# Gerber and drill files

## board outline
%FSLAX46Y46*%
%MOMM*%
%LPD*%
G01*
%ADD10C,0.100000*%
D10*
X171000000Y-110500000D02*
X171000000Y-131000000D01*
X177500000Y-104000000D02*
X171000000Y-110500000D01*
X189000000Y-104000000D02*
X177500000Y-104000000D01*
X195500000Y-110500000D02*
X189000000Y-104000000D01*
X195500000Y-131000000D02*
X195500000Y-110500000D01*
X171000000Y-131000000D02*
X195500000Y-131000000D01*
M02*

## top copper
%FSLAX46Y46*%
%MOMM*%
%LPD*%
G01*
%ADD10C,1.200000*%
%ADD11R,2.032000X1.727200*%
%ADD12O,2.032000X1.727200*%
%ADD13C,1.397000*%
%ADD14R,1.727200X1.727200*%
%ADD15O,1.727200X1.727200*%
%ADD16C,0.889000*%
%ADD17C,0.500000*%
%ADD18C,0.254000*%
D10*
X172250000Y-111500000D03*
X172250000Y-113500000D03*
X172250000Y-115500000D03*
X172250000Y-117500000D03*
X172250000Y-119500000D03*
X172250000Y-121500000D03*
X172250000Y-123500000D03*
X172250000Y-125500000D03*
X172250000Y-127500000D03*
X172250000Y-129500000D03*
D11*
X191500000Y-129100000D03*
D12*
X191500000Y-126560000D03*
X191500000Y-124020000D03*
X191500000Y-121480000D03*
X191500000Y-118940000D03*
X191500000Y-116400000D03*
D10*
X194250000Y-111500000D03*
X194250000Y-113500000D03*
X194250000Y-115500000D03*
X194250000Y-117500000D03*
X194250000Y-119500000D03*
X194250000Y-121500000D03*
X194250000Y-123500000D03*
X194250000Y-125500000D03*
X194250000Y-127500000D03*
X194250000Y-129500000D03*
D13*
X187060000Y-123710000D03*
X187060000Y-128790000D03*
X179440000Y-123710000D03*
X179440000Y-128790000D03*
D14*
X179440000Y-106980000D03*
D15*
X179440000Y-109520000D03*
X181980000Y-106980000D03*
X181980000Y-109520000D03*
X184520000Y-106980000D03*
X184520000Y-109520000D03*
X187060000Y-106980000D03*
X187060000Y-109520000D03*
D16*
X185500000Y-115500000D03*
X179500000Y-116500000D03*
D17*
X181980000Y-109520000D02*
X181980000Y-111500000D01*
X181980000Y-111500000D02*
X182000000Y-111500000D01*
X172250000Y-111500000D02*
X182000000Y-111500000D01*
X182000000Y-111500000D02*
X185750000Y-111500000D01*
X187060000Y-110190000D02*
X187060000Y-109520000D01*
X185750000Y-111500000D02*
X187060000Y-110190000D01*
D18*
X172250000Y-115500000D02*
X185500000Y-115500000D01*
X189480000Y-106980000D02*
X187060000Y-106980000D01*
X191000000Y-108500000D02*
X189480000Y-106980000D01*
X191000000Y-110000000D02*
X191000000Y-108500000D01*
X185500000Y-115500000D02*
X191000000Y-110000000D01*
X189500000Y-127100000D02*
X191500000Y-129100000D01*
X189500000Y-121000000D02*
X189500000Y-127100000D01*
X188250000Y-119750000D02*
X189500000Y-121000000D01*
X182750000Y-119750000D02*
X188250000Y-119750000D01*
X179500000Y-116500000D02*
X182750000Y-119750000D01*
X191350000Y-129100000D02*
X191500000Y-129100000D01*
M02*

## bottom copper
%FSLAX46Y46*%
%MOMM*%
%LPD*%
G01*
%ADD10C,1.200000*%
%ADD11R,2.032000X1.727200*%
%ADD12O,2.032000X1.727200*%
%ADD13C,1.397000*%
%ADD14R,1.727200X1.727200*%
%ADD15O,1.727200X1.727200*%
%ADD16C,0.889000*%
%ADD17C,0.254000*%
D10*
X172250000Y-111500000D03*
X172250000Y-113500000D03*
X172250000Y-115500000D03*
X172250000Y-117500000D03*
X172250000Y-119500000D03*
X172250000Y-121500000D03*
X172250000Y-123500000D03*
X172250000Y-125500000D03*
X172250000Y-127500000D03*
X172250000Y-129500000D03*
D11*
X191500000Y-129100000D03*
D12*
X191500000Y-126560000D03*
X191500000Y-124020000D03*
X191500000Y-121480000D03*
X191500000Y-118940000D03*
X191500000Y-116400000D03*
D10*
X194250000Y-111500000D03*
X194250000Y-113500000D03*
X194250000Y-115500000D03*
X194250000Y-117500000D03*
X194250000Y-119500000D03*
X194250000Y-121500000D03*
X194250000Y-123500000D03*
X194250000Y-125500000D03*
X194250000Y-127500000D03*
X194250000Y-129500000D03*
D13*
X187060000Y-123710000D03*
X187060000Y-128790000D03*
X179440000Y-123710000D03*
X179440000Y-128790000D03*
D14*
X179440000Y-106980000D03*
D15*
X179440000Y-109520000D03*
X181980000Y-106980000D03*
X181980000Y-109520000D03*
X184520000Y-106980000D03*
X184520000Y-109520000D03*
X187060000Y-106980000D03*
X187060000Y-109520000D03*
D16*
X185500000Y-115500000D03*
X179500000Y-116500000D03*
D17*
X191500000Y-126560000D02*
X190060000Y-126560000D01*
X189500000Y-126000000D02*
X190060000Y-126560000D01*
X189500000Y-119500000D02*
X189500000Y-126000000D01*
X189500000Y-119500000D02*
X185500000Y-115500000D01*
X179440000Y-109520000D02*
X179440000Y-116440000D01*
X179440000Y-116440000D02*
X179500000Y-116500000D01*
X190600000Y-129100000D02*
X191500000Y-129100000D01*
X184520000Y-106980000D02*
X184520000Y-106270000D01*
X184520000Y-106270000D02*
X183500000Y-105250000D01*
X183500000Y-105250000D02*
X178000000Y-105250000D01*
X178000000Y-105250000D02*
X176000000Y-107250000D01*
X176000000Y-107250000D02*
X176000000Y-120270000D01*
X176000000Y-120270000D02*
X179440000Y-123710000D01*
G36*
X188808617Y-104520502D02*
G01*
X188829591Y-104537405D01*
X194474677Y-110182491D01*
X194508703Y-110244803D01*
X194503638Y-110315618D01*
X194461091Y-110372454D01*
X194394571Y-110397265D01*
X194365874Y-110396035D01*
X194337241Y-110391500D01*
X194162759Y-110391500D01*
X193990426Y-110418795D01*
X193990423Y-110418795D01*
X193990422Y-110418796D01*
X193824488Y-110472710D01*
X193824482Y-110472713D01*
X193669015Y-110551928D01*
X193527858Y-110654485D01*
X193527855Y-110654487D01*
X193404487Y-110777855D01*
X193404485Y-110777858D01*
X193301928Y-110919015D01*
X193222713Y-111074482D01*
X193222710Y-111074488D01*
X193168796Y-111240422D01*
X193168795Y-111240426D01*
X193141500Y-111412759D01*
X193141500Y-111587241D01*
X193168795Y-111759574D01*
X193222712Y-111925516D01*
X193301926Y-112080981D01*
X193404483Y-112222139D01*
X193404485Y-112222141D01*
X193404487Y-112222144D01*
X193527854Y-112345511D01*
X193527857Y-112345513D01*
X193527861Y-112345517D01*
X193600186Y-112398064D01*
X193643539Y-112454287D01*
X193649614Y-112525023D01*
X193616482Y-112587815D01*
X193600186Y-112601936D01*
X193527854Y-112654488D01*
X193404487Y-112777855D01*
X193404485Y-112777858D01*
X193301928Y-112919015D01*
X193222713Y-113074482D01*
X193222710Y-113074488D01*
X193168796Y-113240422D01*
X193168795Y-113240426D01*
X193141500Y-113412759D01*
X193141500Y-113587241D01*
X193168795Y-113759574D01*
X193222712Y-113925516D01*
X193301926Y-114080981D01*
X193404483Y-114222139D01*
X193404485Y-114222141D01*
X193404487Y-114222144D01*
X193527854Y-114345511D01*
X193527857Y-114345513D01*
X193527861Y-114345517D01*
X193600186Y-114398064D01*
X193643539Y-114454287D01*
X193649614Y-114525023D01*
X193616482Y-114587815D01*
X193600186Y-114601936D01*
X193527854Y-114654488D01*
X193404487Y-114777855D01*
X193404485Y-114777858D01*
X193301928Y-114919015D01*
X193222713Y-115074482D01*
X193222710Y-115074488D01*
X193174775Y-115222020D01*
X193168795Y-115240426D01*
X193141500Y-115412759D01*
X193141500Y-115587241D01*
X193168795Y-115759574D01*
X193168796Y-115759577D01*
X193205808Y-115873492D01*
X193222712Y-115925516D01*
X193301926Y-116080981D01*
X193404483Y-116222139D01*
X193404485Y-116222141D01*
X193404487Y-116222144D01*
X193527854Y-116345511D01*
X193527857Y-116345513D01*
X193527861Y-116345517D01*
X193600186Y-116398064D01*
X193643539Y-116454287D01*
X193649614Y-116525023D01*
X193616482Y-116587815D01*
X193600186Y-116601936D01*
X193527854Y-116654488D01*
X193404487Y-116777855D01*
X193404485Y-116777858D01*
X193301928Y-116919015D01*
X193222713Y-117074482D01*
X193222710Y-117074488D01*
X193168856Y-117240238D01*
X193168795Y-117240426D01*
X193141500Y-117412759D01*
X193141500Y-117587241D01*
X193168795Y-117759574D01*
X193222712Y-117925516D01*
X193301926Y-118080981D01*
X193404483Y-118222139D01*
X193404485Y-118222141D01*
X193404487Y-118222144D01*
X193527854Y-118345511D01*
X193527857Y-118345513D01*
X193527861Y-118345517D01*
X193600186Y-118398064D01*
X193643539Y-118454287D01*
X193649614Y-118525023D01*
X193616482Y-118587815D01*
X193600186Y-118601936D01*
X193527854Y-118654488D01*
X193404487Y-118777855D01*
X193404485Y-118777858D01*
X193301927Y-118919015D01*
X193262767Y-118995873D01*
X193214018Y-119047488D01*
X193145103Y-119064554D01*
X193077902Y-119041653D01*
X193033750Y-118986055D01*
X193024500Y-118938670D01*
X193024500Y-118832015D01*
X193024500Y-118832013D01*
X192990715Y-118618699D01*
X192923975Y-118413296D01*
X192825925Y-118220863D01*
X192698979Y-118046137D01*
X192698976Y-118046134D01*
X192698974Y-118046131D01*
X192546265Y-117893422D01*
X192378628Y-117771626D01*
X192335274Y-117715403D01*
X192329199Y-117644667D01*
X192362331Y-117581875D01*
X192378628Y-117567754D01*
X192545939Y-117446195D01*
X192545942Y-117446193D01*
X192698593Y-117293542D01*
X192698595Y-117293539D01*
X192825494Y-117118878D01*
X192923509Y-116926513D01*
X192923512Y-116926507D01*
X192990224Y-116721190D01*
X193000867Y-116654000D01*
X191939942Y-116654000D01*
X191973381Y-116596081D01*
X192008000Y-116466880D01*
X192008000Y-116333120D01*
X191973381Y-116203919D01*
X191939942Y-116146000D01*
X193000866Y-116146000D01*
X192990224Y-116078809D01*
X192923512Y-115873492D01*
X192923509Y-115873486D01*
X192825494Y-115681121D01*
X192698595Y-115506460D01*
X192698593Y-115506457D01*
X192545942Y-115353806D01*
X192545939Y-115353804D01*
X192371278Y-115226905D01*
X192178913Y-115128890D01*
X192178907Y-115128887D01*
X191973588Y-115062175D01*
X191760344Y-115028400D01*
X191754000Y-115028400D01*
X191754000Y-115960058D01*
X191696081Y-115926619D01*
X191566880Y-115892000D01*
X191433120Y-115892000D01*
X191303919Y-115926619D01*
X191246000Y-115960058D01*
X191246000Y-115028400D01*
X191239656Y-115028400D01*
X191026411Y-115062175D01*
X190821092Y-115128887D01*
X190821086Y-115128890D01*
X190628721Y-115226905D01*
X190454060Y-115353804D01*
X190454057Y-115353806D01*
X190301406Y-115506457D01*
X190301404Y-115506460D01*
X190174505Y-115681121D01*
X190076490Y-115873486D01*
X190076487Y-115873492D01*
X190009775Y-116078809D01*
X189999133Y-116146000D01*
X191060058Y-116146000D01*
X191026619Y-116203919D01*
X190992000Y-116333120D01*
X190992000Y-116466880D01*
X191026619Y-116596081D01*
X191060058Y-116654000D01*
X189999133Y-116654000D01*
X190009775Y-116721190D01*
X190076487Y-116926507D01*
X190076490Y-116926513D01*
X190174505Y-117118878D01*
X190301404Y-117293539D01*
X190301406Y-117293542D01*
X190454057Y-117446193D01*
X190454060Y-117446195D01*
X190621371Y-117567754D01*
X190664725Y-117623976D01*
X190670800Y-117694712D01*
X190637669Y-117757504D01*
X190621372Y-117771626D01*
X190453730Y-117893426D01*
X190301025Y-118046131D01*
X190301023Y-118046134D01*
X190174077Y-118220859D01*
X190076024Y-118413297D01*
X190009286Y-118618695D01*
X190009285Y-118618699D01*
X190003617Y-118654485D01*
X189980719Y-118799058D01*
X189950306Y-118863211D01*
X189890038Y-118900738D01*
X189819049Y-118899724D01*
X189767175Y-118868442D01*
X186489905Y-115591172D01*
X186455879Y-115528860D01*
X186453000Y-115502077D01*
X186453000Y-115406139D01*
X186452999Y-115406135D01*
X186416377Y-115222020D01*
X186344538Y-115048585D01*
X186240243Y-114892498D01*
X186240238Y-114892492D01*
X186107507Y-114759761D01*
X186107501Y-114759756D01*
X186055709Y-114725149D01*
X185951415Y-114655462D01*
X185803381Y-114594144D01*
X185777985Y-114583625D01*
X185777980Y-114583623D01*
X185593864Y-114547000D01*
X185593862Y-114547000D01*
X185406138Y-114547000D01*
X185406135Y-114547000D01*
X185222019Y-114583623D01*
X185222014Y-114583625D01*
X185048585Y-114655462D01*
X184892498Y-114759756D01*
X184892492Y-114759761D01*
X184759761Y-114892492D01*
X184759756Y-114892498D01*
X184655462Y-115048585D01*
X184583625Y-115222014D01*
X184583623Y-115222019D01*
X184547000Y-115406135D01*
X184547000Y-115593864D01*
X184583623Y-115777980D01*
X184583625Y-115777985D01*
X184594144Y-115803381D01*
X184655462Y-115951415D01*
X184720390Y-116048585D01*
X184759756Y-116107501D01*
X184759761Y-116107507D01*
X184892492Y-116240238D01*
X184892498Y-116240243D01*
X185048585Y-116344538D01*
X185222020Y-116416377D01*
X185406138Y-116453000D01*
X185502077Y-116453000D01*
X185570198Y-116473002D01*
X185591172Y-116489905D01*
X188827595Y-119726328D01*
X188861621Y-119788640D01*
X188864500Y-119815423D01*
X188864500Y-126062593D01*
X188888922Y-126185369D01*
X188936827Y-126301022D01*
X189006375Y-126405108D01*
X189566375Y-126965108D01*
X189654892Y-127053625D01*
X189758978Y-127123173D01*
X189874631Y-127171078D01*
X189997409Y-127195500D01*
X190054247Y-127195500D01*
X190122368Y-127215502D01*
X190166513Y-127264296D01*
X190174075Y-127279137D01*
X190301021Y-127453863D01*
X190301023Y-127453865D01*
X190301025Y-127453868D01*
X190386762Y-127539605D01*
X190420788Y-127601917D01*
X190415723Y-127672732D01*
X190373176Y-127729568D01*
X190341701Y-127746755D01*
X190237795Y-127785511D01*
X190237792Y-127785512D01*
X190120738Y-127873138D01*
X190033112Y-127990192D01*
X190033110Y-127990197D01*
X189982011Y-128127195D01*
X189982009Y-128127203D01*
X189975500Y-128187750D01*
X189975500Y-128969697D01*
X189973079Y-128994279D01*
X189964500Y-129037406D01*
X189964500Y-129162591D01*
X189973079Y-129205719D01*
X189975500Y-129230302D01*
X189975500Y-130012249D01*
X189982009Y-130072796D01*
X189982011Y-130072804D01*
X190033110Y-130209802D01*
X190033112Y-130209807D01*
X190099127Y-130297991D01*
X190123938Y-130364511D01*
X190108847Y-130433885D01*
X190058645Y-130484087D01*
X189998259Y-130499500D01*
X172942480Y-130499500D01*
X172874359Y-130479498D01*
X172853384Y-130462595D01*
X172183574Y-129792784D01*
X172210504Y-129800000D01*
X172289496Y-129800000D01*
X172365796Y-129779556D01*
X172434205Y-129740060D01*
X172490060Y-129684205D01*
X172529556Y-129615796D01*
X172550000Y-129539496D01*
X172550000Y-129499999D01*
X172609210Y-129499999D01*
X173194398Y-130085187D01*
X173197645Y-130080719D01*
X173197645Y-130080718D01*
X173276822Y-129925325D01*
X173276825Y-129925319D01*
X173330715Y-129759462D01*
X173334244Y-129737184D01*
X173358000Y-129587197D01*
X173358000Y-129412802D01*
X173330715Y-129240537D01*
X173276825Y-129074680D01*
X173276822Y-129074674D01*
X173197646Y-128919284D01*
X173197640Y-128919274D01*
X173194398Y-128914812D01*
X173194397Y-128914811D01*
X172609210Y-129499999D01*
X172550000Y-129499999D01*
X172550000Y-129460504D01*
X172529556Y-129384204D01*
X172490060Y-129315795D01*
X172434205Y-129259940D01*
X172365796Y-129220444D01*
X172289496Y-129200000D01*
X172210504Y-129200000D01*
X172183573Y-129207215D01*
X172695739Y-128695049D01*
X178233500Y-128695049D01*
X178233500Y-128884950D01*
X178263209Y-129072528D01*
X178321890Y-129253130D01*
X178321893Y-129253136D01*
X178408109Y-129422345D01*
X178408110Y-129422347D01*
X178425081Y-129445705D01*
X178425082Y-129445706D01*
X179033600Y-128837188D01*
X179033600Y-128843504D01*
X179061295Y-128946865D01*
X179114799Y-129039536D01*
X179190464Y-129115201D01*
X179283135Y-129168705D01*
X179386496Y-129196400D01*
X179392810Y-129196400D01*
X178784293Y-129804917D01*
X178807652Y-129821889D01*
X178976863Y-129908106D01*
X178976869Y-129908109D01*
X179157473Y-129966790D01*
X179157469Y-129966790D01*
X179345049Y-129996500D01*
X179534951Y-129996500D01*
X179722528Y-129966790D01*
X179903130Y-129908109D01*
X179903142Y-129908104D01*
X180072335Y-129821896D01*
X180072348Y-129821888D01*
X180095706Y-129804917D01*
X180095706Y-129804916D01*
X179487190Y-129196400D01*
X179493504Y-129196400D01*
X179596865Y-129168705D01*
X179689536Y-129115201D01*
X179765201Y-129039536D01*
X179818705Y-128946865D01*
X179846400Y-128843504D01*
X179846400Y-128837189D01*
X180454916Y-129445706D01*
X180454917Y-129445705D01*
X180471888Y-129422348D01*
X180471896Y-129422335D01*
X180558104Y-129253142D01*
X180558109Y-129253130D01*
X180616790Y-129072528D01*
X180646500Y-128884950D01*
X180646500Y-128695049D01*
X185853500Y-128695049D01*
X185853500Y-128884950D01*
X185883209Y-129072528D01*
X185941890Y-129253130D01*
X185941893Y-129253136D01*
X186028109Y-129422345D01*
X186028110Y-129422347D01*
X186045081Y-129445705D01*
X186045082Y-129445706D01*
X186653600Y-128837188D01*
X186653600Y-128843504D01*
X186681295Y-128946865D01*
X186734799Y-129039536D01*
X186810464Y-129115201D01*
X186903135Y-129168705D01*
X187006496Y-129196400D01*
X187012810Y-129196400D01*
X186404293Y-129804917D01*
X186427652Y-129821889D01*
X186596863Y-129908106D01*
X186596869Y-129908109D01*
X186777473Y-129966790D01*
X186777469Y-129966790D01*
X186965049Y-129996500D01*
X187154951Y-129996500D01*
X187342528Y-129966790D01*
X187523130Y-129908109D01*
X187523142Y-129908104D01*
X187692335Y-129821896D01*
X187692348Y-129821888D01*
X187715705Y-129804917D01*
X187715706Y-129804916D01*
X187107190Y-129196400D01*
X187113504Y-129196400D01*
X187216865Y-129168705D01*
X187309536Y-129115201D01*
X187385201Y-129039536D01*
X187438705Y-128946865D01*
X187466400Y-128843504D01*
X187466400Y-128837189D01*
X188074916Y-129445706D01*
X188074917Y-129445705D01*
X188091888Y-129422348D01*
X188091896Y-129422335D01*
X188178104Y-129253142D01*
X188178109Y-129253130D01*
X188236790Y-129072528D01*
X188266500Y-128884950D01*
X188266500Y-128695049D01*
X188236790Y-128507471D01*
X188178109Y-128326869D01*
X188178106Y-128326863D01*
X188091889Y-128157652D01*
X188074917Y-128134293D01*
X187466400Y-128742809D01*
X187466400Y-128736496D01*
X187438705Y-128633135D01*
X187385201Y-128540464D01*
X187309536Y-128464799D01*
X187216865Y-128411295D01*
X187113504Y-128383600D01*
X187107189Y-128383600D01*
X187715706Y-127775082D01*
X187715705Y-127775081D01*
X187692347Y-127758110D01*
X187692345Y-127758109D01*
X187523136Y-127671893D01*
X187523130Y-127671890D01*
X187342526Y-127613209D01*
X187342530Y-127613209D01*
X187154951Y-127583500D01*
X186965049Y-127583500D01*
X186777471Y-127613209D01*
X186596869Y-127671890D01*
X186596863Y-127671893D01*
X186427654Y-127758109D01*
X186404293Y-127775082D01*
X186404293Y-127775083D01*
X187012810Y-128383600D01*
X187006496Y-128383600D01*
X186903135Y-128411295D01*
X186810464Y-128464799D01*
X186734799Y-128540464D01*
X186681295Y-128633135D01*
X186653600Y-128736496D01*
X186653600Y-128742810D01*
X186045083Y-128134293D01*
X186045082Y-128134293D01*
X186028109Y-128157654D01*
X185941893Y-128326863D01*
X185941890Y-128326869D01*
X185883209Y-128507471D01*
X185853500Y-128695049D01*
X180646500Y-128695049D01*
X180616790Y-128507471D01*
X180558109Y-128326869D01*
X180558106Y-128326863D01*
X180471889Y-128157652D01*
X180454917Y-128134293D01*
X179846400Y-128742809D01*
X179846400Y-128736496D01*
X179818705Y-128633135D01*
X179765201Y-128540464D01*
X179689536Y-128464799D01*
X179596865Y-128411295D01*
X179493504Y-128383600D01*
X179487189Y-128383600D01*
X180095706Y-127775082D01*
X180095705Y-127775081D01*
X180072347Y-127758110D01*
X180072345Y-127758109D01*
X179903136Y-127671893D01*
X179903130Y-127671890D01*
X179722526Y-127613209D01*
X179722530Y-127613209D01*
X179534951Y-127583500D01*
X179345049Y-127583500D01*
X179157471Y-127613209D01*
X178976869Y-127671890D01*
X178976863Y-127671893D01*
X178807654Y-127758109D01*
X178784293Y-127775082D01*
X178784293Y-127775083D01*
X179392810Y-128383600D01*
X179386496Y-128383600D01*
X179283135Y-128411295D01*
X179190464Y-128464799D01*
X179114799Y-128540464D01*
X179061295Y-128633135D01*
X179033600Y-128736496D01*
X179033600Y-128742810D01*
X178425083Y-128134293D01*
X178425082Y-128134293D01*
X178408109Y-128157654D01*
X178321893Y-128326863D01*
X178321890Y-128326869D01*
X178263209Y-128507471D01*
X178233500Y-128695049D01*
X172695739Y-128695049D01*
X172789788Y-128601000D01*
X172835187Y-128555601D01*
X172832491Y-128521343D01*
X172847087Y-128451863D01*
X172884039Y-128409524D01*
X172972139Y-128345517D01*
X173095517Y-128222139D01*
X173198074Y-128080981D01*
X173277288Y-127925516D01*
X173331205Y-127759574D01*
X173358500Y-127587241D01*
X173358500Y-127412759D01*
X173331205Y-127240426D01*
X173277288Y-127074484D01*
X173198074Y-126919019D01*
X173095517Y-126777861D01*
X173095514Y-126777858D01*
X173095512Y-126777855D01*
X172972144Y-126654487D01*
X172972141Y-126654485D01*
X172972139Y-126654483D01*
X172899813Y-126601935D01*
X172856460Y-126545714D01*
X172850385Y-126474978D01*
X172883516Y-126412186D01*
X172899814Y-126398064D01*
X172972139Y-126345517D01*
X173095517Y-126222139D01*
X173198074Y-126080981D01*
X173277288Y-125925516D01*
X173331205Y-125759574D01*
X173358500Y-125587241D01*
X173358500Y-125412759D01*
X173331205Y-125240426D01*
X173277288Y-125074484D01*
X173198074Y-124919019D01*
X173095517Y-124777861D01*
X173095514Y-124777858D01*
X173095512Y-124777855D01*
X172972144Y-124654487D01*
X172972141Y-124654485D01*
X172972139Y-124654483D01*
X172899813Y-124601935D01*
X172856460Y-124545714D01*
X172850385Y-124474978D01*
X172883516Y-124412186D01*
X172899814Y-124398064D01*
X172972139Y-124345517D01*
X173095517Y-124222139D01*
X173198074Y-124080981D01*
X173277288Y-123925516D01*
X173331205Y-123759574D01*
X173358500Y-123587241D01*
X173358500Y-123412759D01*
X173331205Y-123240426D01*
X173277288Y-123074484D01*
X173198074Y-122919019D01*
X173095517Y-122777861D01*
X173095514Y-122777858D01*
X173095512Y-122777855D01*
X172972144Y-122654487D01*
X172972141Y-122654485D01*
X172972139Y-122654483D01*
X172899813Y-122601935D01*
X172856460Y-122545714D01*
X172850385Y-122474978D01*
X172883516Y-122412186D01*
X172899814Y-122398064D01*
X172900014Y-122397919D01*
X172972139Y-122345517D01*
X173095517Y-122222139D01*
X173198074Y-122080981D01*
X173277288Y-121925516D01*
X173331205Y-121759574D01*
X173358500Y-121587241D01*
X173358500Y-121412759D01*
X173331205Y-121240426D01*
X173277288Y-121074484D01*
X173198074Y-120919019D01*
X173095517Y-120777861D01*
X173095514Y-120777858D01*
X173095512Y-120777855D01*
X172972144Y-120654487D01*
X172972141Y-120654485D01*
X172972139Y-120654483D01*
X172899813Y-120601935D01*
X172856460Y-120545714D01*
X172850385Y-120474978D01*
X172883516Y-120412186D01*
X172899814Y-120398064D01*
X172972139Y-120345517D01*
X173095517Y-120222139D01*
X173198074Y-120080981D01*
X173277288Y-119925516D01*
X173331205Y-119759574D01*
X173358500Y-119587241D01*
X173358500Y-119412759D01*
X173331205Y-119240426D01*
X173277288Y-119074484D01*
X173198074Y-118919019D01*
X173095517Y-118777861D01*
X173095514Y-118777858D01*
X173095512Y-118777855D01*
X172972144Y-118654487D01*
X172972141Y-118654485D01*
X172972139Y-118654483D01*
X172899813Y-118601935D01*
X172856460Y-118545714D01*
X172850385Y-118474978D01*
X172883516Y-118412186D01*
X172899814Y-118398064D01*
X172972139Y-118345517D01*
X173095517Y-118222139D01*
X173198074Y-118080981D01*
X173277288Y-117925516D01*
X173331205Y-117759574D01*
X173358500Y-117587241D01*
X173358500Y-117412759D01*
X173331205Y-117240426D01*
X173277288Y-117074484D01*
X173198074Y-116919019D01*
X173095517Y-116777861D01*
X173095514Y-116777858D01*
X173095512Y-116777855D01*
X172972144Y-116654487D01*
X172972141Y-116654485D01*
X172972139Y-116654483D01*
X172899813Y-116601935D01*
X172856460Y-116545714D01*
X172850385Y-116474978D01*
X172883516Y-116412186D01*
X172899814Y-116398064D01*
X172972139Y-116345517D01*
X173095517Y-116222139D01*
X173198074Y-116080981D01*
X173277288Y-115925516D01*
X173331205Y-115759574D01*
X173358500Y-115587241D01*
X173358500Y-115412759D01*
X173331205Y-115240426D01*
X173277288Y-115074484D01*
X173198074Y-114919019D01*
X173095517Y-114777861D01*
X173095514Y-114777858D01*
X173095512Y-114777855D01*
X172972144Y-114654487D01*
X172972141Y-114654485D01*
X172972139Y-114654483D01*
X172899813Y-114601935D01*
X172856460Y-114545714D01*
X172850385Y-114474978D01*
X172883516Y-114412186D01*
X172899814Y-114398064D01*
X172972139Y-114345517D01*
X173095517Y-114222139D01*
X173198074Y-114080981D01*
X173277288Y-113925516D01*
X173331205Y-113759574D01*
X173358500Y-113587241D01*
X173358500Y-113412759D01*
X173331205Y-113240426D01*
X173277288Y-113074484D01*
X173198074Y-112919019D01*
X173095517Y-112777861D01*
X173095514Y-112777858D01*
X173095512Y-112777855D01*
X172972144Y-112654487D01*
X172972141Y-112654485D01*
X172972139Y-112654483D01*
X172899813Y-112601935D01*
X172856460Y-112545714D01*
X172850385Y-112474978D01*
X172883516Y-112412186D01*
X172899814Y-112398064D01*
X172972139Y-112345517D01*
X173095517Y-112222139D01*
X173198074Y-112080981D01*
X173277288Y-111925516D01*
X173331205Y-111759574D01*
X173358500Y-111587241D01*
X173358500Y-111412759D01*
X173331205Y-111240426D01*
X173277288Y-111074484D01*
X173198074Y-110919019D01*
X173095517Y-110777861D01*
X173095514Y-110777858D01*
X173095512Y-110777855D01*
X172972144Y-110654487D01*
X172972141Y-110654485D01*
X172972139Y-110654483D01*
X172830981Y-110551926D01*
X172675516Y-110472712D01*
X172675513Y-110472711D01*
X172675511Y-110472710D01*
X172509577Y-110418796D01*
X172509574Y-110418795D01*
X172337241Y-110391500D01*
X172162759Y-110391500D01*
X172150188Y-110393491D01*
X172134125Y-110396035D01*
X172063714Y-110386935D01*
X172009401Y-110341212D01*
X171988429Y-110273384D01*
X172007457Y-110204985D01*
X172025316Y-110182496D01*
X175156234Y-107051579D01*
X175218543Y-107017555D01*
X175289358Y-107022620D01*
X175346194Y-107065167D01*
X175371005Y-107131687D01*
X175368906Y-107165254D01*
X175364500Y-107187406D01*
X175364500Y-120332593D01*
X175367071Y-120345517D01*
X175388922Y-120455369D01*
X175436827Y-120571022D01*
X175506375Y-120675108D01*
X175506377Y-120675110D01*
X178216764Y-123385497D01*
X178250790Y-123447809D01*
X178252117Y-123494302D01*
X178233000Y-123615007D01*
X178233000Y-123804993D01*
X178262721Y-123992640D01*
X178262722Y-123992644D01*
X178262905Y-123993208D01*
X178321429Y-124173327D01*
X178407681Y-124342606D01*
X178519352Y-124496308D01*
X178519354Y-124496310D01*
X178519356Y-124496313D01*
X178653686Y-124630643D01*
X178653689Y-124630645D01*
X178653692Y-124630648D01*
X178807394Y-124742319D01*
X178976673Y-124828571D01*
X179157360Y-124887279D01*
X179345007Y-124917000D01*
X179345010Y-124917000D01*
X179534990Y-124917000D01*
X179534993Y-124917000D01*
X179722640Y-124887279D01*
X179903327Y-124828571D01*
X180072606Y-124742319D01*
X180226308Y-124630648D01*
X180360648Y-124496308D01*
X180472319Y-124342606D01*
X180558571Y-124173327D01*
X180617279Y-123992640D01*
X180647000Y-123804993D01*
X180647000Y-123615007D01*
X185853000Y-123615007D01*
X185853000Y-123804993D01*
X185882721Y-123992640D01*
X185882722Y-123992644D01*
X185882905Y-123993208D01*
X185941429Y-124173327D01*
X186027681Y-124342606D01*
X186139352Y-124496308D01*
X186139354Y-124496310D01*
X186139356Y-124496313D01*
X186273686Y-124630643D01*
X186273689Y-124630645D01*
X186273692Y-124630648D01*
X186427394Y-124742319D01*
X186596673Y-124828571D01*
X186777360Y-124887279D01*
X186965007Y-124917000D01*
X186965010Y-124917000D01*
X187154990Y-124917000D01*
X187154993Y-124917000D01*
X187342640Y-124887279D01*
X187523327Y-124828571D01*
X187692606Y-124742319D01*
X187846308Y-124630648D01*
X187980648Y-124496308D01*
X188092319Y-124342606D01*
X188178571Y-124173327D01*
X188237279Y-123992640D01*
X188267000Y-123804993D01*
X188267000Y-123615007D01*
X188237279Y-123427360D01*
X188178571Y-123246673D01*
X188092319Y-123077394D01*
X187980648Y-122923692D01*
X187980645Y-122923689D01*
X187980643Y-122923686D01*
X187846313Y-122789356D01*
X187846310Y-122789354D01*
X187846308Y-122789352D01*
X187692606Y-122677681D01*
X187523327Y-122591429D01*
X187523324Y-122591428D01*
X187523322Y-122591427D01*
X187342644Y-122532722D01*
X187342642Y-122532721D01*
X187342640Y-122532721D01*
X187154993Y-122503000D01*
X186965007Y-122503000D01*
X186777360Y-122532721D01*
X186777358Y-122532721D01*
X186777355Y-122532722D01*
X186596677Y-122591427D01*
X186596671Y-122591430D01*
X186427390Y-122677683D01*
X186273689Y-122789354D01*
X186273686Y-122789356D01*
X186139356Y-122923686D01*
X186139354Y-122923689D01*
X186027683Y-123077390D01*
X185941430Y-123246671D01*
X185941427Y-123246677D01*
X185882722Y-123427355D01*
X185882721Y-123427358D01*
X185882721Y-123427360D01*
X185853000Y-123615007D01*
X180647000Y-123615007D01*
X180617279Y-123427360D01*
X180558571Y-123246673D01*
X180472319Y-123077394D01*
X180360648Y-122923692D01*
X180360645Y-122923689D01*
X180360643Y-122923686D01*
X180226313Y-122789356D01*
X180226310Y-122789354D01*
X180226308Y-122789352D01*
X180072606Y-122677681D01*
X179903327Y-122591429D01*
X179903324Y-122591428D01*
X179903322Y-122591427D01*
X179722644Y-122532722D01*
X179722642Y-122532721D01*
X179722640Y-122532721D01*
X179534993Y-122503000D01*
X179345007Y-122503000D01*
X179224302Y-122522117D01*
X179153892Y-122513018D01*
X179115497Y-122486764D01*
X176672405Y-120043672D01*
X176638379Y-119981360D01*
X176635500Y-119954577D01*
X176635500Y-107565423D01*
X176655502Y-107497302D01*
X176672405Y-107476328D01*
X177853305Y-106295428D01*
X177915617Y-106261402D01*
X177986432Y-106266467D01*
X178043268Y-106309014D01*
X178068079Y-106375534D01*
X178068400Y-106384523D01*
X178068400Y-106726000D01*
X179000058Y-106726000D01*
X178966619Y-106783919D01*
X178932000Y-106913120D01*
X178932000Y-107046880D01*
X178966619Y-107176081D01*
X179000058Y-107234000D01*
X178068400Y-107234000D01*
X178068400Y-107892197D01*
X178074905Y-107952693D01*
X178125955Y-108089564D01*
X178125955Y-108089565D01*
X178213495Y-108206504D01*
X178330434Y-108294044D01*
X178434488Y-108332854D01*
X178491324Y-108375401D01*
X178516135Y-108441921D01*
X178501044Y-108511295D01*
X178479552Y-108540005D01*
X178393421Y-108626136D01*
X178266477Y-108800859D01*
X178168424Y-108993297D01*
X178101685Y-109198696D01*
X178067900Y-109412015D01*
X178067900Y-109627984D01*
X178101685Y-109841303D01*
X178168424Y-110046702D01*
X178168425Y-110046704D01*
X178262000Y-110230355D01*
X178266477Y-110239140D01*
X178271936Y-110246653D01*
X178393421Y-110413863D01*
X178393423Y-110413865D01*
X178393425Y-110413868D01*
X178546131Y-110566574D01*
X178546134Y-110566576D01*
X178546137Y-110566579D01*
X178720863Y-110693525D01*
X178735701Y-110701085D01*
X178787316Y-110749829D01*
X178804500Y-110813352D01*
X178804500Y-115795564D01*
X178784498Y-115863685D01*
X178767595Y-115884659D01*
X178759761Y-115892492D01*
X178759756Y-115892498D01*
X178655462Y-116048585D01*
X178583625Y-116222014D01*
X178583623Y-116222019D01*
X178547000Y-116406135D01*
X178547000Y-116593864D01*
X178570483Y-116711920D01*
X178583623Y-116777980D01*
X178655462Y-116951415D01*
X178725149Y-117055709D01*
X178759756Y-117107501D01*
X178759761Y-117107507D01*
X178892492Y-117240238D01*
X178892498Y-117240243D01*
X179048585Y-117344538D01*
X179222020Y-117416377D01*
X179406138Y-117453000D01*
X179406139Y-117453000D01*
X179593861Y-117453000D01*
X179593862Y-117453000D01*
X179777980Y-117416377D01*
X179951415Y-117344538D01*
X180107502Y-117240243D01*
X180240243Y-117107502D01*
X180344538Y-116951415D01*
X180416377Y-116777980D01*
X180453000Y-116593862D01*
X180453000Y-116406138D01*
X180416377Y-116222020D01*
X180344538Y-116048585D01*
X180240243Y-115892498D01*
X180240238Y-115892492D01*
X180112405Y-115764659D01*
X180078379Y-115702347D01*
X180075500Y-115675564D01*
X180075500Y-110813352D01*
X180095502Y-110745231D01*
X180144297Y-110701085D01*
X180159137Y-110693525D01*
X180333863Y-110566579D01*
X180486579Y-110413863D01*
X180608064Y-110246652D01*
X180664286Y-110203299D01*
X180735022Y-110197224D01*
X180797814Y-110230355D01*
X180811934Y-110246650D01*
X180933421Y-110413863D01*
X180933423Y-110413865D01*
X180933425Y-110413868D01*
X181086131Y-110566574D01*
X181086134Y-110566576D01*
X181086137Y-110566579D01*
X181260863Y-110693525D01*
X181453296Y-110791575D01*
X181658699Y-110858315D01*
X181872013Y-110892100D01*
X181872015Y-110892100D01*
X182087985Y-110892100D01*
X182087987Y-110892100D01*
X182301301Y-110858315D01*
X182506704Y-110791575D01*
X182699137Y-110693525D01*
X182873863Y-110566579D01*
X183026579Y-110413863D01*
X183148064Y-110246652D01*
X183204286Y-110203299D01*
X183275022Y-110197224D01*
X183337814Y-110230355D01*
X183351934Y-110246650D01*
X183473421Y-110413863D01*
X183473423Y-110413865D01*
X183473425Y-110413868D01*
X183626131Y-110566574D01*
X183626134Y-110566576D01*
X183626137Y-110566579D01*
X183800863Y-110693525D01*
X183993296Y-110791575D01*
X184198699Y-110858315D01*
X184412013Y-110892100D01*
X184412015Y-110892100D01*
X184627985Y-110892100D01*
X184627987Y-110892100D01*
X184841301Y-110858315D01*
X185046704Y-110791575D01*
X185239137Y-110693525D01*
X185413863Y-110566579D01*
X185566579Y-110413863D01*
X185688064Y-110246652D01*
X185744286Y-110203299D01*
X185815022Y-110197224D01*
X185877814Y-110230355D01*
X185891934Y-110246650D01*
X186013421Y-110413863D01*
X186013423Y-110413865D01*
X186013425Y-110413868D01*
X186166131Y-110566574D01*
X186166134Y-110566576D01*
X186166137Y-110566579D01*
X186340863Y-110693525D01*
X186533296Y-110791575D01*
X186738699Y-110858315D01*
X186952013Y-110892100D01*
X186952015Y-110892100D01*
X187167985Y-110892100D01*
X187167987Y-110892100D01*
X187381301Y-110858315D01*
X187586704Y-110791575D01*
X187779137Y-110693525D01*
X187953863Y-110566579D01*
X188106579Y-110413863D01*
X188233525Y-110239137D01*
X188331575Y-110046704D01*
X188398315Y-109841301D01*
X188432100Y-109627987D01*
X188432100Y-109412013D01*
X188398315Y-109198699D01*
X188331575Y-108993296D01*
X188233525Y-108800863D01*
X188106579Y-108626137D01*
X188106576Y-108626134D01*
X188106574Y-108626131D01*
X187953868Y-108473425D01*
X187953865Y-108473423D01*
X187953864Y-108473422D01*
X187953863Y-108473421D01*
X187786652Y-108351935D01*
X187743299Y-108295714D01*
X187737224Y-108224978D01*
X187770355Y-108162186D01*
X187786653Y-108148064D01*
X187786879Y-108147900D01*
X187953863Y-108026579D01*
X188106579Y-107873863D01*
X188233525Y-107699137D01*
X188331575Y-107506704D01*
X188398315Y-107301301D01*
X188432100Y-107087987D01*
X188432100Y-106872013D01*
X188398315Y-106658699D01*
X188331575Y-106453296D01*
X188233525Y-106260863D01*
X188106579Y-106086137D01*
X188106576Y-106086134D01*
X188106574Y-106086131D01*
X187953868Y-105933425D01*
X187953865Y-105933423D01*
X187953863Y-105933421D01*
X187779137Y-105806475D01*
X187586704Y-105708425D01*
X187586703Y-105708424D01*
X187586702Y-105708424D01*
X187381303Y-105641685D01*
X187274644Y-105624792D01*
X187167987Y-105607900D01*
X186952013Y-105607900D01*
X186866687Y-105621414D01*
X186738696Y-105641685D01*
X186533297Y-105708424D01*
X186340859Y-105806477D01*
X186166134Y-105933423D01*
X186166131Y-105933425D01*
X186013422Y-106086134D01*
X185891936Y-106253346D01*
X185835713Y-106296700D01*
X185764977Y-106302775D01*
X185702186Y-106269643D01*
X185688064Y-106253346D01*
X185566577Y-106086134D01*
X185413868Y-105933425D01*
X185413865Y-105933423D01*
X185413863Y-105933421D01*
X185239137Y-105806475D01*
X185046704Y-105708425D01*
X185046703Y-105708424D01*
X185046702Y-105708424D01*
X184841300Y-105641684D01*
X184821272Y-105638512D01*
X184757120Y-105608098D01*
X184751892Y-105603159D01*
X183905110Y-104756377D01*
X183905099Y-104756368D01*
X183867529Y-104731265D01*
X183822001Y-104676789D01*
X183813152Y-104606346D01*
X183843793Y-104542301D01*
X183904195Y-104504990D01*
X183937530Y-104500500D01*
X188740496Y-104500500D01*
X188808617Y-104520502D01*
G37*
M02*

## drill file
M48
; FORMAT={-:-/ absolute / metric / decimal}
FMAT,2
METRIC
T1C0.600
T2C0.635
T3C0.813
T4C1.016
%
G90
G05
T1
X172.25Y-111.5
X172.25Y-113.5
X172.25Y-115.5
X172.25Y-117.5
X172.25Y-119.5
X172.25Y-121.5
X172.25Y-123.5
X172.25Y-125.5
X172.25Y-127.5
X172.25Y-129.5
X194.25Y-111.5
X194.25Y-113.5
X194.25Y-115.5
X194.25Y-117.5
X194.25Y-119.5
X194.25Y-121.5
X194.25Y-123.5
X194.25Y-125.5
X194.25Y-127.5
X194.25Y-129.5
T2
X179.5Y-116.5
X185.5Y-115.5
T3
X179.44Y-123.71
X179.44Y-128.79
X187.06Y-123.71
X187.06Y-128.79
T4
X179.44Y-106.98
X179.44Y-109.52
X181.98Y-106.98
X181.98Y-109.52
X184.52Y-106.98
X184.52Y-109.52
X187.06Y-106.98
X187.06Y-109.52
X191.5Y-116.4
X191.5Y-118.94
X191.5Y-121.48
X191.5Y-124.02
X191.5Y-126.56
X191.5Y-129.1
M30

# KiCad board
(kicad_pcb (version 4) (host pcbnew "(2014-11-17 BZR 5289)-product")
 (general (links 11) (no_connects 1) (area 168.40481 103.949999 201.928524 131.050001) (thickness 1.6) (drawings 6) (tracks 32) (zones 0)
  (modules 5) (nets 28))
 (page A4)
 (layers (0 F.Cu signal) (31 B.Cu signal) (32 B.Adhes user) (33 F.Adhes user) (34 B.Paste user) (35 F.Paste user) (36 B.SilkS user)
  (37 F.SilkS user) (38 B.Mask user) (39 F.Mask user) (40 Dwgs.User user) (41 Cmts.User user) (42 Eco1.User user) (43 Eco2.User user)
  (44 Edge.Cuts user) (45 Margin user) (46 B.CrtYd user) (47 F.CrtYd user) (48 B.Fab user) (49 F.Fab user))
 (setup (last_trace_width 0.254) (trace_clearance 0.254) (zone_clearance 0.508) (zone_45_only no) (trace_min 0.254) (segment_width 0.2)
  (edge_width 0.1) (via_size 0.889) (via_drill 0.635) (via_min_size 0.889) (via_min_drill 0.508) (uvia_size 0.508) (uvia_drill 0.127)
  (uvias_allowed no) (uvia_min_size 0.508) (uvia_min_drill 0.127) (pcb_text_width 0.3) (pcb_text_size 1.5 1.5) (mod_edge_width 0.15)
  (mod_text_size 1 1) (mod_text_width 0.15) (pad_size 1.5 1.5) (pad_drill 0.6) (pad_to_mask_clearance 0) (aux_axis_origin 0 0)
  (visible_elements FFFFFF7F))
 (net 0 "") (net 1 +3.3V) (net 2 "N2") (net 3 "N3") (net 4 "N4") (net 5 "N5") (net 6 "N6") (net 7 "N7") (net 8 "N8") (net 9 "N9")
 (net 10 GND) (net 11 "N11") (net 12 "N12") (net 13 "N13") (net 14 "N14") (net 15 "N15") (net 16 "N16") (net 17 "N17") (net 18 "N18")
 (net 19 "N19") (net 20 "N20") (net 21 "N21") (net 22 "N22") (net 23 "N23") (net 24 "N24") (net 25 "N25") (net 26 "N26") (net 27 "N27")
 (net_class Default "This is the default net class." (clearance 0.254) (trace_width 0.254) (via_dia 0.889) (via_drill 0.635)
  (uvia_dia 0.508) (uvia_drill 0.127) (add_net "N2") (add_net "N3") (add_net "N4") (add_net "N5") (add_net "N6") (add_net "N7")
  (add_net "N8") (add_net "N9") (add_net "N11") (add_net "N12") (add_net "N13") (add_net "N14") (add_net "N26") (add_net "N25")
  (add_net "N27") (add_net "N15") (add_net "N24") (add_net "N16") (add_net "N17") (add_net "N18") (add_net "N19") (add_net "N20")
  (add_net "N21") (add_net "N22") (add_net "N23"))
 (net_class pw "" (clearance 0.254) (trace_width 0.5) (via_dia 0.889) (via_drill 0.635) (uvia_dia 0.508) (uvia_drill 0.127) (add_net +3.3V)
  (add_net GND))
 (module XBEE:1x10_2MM (layer F.Cu) (at 172.25 120.5 270)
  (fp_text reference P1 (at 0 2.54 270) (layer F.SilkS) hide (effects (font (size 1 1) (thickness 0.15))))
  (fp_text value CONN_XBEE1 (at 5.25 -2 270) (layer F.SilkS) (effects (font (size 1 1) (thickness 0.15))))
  (pad 1 thru_hole circle (at -9 0 270) (size 1.2 1.2) (drill 0.6) (layers *.Cu *.Mask F.SilkS) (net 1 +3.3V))
  (pad 2 thru_hole circle (at -7 0 270) (size 1.2 1.2) (drill 0.6) (layers *.Cu *.Mask F.SilkS) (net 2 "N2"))
  (pad 3 thru_hole circle (at -5 0 270) (size 1.2 1.2) (drill 0.6) (layers *.Cu *.Mask F.SilkS) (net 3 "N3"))
  (pad 4 thru_hole circle (at -3 0 270) (size 1.2 1.2) (drill 0.6) (layers *.Cu *.Mask F.SilkS) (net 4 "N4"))
  (pad 5 thru_hole circle (at -1 0 270) (size 1.2 1.2) (drill 0.6) (layers *.Cu *.Mask F.SilkS) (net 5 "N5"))
  (pad 6 thru_hole circle (at 1 0 270) (size 1.2 1.2) (drill 0.6) (layers *.Cu *.Mask F.SilkS) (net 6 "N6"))
  (pad 7 thru_hole circle (at 3 0 270) (size 1.2 1.2) (drill 0.6) (layers *.Cu *.Mask F.SilkS) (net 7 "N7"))
  (pad 8 thru_hole circle (at 5 0 270) (size 1.2 1.2) (drill 0.6) (layers *.Cu *.Mask F.SilkS) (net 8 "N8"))
  (pad 9 thru_hole circle (at 7 0 270) (size 1.2 1.2) (drill 0.6) (layers *.Cu *.Mask F.SilkS) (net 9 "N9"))
  (pad 10 thru_hole circle (at 9 0 270) (size 1.2 1.2) (drill 0.6) (layers *.Cu *.Mask F.SilkS) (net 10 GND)))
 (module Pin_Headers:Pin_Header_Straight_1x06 (layer F.Cu) (at 191.5 122.75 90)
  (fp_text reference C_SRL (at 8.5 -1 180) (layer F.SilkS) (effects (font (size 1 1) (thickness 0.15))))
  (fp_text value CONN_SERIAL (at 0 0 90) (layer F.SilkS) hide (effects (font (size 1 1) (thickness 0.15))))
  (pad 1 thru_hole rect (at -6.35 0 90) (size 1.7272 2.032) (drill 1.016) (layers *.Cu *.Mask F.SilkS) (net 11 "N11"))
  (pad 2 thru_hole oval (at -3.81 0 90) (size 1.7272 2.032) (drill 1.016) (layers *.Cu *.Mask F.SilkS) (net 3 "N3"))
  (pad 3 thru_hole oval (at -1.27 0 90) (size 1.7272 2.032) (drill 1.016) (layers *.Cu *.Mask F.SilkS) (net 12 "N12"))
  (pad 4 thru_hole oval (at 1.27 0 90) (size 1.7272 2.032) (drill 1.016) (layers *.Cu *.Mask F.SilkS) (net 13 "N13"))
  (pad 5 thru_hole oval (at 3.81 0 90) (size 1.7272 2.032) (drill 1.016) (layers *.Cu *.Mask F.SilkS) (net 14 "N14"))
  (pad 6 thru_hole oval (at 6.35 0 90) (size 1.7272 2.032) (drill 1.016) (layers *.Cu *.Mask F.SilkS) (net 10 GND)))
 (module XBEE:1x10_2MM (layer F.Cu) (at 194.25 120.5 270)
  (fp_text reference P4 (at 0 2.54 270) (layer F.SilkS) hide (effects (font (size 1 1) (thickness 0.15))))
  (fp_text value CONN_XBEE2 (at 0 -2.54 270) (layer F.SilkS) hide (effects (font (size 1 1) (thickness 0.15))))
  (pad 1 thru_hole circle (at -9 0 270) (size 1.2 1.2) (drill 0.6) (layers *.Cu *.Mask F.SilkS) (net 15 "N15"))
  (pad 2 thru_hole circle (at -7 0 270) (size 1.2 1.2) (drill 0.6) (layers *.Cu *.Mask F.SilkS) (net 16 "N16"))
  (pad 3 thru_hole circle (at -5 0 270) (size 1.2 1.2) (drill 0.6) (layers *.Cu *.Mask F.SilkS) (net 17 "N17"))
  (pad 4 thru_hole circle (at -3 0 270) (size 1.2 1.2) (drill 0.6) (layers *.Cu *.Mask F.SilkS) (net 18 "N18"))
  (pad 5 thru_hole circle (at -1 0 270) (size 1.2 1.2) (drill 0.6) (layers *.Cu *.Mask F.SilkS) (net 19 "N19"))
  (pad 6 thru_hole circle (at 1 0 270) (size 1.2 1.2) (drill 0.6) (layers *.Cu *.Mask F.SilkS) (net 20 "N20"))
  (pad 7 thru_hole circle (at 3 0 270) (size 1.2 1.2) (drill 0.6) (layers *.Cu *.Mask F.SilkS) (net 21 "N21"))
  (pad 8 thru_hole circle (at 5 0 270) (size 1.2 1.2) (drill 0.6) (layers *.Cu *.Mask F.SilkS) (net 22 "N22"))
  (pad 9 thru_hole circle (at 7 0 270) (size 1.2 1.2) (drill 0.6) (layers *.Cu *.Mask F.SilkS) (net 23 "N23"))
  (pad 10 thru_hole circle (at 9 0 270) (size 1.2 1.2) (drill 0.6) (layers *.Cu *.Mask F.SilkS) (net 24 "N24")))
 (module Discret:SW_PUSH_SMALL (layer F.Cu) (at 183.25 126.25)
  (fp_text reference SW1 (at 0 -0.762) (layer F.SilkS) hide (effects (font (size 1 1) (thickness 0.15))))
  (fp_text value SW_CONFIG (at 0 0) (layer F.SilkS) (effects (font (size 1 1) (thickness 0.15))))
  (pad 1 thru_hole circle (at 3.81 -2.54) (size 1.397 1.397) (drill 0.8128) (layers *.Cu *.Mask F.SilkS) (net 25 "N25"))
  (pad 2 thru_hole circle (at 3.81 2.54) (size 1.397 1.397) (drill 0.8128) (layers *.Cu *.Mask F.SilkS) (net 10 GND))
  (pad 1 thru_hole circle (at -3.81 -2.54) (size 1.397 1.397) (drill 0.8128) (layers *.Cu *.Mask F.SilkS) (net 25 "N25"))
  (pad 2 thru_hole circle (at -3.81 2.54) (size 1.397 1.397) (drill 0.8128) (layers *.Cu *.Mask F.SilkS) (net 10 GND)))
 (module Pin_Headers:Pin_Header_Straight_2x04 (layer B.Cu) (at 183.25 108.25)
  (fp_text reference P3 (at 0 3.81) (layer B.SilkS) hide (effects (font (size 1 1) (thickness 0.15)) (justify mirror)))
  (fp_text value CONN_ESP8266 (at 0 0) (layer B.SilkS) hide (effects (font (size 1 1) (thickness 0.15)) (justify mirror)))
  (pad 1 thru_hole rect (at -3.81 -1.27) (size 1.7272 1.7272) (drill 1.016) (layers *.Cu *.Mask B.SilkS) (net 10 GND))
  (pad 2 thru_hole oval (at -3.81 1.27) (size 1.7272 1.7272) (drill 1.016) (layers *.Cu *.Mask B.SilkS) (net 11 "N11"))
  (pad 3 thru_hole oval (at -1.27 -1.27) (size 1.7272 1.7272) (drill 1.016) (layers *.Cu *.Mask B.SilkS) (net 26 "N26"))
  (pad 4 thru_hole oval (at -1.27 1.27) (size 1.7272 1.7272) (drill 1.016) (layers *.Cu *.Mask B.SilkS) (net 1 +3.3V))
  (pad 5 thru_hole oval (at 1.27 -1.27) (size 1.7272 1.7272) (drill 1.016) (layers *.Cu *.Mask B.SilkS) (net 25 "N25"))
  (pad 6 thru_hole oval (at 1.27 1.27) (size 1.7272 1.7272) (drill 1.016) (layers *.Cu *.Mask B.SilkS) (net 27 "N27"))
  (pad 7 thru_hole oval (at 3.81 -1.27) (size 1.7272 1.7272) (drill 1.016) (layers *.Cu *.Mask B.SilkS) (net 3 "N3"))
  (pad 8 thru_hole oval (at 3.81 1.27) (size 1.7272 1.7272) (drill 1.016) (layers *.Cu *.Mask B.SilkS) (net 1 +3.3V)))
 (gr_line (start 171 110.5) (end 171 131) (angle 90) (layer Edge.Cuts) (width 0.1))
 (gr_line (start 177.5 104) (end 171 110.5) (angle 90) (layer Edge.Cuts) (width 0.1))
 (gr_line (start 189 104) (end 177.5 104) (angle 90) (layer Edge.Cuts) (width 0.1))
 (gr_line (start 195.5 110.5) (end 189 104) (angle 90) (layer Edge.Cuts) (width 0.1))
 (gr_line (start 195.5 131) (end 195.5 110.5) (angle 90) (layer Edge.Cuts) (width 0.1))
 (gr_line (start 171 131) (end 195.5 131) (angle 90) (layer Edge.Cuts) (width 0.1))
 (segment (start 181.98 109.52) (end 181.98 111.5) (width 0.5) (layer F.Cu) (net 1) (status 400000))
 (segment (start 181.98 111.5) (end 182 111.5) (width 0.5) (layer F.Cu) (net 1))
 (segment (start 172.25 111.5) (end 182 111.5) (width 0.5) (layer F.Cu) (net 1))
 (segment (start 182 111.5) (end 185.75 111.5) (width 0.5) (layer F.Cu) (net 1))
 (segment (start 187.06 110.19) (end 187.06 109.52) (width 0.5) (layer F.Cu) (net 1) (status 30))
 (segment (start 185.75 111.5) (end 187.06 110.19) (width 0.5) (layer F.Cu) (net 1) (status 20))
 (via (at 185.5 115.5) (size 0.889) (layers F.Cu B.Cu) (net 3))
 (segment (start 191.5 126.56) (end 190.06 126.56) (width 0.254) (layer B.Cu) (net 3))
 (segment (start 189.5 126) (end 190.06 126.56) (width 0.254) (layer B.Cu) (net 3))
 (segment (start 189.5 119.5) (end 189.5 126) (width 0.254) (layer B.Cu) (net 3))
 (segment (start 189.5 119.5) (end 185.5 115.5) (width 0.254) (layer B.Cu) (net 3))
 (segment (start 172.25 115.5) (end 185.5 115.5) (width 0.254) (layer F.Cu) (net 3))
 (segment (start 189.48 106.98) (end 187.06 106.98) (width 0.254) (layer F.Cu) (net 3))
 (segment (start 191 108.5) (end 189.48 106.98) (width 0.254) (layer F.Cu) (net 3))
 (segment (start 191 110) (end 191 108.5) (width 0.254) (layer F.Cu) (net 3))
 (segment (start 185.5 115.5) (end 191 110) (width 0.254) (layer F.Cu) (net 3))
 (segment (start 179.44 109.52) (end 179.44 116.44) (width 0.254) (layer B.Cu) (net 11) (status 400000))
 (segment (start 189.5 127.1) (end 191.5 129.1) (width 0.254) (layer F.Cu) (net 11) (status 800000))
 (segment (start 189.5 121) (end 189.5 127.1) (width 0.254) (layer F.Cu) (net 11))
 (segment (start 188.25 119.75) (end 189.5 121) (width 0.254) (layer F.Cu) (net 11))
 (segment (start 182.75 119.75) (end 188.25 119.75) (width 0.254) (layer F.Cu) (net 11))
 (segment (start 179.5 116.5) (end 182.75 119.75) (width 0.254) (layer F.Cu) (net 11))
 (via (at 179.5 116.5) (size 0.889) (layers F.Cu B.Cu) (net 11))
 (segment (start 179.44 116.44) (end 179.5 116.5) (width 0.254) (layer B.Cu) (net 11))
 (segment (start 191.35 129.1) (end 191.5 129.1) (width 0.254) (layer F.Cu) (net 11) (status C00000))
 (segment (start 190.6 129.1) (end 191.5 129.1) (width 0.254) (layer B.Cu) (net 11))
 (segment (start 184.52 106.98) (end 184.52 106.27) (width 0.254) (layer B.Cu) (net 25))
 (segment (start 184.52 106.27) (end 183.5 105.25) (width 0.254) (layer B.Cu) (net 25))
 (segment (start 183.5 105.25) (end 178 105.25) (width 0.254) (layer B.Cu) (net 25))
 (segment (start 178 105.25) (end 176 107.25) (width 0.254) (layer B.Cu) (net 25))
 (segment (start 176 107.25) (end 176 120.27) (width 0.254) (layer B.Cu) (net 25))
 (segment (start 176 120.27) (end 179.44 123.71) (width 0.254) (layer B.Cu) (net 25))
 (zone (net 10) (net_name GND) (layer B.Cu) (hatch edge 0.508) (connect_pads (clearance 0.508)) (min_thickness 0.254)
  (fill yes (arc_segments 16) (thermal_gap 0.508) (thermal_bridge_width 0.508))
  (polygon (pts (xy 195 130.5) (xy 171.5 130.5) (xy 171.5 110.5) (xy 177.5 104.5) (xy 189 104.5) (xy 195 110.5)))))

